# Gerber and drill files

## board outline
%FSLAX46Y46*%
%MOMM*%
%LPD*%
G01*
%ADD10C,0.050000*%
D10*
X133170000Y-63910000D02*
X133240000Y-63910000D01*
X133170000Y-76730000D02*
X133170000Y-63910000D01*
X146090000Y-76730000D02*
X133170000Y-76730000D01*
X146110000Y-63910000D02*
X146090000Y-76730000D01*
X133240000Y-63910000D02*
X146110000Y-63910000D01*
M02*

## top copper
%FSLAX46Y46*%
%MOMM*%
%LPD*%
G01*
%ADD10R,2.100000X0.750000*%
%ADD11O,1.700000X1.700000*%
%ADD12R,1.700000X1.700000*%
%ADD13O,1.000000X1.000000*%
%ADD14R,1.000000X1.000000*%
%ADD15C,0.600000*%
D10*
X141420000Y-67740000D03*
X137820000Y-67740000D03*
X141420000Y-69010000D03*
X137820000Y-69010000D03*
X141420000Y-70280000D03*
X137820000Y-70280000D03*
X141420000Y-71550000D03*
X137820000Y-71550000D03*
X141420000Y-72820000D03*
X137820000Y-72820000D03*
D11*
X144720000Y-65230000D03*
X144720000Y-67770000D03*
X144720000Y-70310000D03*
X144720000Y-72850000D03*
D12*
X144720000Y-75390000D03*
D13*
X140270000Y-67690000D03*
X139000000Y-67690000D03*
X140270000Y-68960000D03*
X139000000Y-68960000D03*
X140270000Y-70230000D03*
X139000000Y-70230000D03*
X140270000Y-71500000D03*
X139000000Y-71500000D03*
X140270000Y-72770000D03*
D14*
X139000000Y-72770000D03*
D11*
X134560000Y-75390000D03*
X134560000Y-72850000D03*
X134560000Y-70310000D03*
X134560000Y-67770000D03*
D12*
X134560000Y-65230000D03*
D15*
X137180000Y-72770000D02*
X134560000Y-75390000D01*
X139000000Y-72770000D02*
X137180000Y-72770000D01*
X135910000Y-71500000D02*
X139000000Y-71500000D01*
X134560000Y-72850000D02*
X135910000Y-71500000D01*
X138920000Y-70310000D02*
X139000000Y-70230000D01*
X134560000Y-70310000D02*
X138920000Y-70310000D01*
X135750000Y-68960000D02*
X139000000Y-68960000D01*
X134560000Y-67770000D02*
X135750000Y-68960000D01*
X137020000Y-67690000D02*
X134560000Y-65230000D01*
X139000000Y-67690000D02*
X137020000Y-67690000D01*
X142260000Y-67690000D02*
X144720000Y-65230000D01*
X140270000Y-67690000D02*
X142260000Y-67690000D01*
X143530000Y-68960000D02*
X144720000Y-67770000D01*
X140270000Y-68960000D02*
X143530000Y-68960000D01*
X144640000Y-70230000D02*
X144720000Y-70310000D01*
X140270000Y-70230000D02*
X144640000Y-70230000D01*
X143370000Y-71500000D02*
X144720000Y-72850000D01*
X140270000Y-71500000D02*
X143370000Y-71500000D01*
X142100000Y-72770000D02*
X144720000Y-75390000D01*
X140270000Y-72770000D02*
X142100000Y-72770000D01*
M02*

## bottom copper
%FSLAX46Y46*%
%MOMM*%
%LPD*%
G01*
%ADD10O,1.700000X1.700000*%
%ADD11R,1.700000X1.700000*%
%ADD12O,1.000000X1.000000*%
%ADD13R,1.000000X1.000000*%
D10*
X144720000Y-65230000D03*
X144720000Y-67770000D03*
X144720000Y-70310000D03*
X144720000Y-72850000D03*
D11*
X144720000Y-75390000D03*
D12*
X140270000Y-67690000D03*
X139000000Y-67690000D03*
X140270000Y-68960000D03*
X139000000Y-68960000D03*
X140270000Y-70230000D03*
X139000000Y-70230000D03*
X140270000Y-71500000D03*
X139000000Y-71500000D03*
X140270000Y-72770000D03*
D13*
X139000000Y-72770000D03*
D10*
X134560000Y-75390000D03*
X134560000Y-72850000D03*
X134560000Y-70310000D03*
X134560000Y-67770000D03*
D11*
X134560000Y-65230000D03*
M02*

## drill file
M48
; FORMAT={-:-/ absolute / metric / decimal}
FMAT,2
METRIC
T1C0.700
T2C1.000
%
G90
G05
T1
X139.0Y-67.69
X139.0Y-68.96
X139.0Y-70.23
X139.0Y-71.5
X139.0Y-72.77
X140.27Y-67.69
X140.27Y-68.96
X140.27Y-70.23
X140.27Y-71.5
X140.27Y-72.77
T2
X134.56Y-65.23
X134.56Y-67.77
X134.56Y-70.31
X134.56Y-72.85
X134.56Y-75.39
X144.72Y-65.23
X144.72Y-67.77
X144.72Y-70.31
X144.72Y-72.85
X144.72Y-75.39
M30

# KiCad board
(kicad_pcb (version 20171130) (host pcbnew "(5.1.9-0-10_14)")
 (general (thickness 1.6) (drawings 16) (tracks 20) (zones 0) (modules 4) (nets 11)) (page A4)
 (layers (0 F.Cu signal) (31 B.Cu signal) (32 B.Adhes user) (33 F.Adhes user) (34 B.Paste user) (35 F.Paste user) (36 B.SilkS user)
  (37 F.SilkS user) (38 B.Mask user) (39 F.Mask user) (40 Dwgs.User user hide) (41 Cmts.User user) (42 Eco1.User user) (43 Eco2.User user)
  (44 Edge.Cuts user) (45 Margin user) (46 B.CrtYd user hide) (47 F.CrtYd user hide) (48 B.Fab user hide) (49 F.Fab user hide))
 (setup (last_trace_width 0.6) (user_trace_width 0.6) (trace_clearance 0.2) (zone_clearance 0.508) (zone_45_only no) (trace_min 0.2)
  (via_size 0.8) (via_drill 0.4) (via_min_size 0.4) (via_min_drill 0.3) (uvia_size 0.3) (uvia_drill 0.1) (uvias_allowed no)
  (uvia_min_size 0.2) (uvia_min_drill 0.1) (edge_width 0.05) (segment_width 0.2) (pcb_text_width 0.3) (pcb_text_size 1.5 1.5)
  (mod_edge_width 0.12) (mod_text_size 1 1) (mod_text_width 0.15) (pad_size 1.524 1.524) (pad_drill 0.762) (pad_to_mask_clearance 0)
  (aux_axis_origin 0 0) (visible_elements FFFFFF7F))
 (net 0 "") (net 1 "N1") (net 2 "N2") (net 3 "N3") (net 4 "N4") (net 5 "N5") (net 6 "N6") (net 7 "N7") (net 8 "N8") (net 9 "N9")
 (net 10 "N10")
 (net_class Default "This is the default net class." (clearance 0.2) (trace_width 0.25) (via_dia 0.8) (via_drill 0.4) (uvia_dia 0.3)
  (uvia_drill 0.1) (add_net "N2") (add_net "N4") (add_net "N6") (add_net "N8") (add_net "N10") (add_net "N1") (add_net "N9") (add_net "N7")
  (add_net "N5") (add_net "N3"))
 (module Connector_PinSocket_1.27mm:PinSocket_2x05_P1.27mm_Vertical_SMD (layer F.Cu) (at 139.62 70.28 180)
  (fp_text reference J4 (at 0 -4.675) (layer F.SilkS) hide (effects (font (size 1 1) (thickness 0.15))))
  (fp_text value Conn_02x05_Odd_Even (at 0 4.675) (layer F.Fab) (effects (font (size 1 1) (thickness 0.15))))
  (pad 10 smd rect (at -1.8 2.54 180) (size 2.1 0.75) (layers F.Cu F.Paste F.Mask) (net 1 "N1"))
  (pad 9 smd rect (at 1.8 2.54 180) (size 2.1 0.75) (layers F.Cu F.Paste F.Mask) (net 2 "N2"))
  (pad 8 smd rect (at -1.8 1.27 180) (size 2.1 0.75) (layers F.Cu F.Paste F.Mask) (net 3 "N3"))
  (pad 7 smd rect (at 1.8 1.27 180) (size 2.1 0.75) (layers F.Cu F.Paste F.Mask) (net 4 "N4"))
  (pad 6 smd rect (at -1.8 0 180) (size 2.1 0.75) (layers F.Cu F.Paste F.Mask) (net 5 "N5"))
  (pad 5 smd rect (at 1.8 0 180) (size 2.1 0.75) (layers F.Cu F.Paste F.Mask) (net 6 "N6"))
  (pad 4 smd rect (at -1.8 -1.27 180) (size 2.1 0.75) (layers F.Cu F.Paste F.Mask) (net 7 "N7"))
  (pad 3 smd rect (at 1.8 -1.27 180) (size 2.1 0.75) (layers F.Cu F.Paste F.Mask) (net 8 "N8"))
  (pad 2 smd rect (at -1.8 -2.54 180) (size 2.1 0.75) (layers F.Cu F.Paste F.Mask) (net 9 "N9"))
  (pad 1 smd rect (at 1.8 -2.54 180) (size 2.1 0.75) (layers F.Cu F.Paste F.Mask) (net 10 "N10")))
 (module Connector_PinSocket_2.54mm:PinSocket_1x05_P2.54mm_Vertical (layer F.Cu) (at 144.72 75.39 180)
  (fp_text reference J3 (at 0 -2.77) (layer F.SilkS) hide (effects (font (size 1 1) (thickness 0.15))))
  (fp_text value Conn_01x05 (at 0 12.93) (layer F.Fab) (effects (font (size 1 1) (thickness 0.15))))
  (pad 5 thru_hole oval (at 0 10.16 180) (size 1.7 1.7) (drill 1) (layers *.Cu *.Mask) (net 1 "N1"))
  (pad 4 thru_hole oval (at 0 7.62 180) (size 1.7 1.7) (drill 1) (layers *.Cu *.Mask) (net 3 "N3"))
  (pad 3 thru_hole oval (at 0 5.08 180) (size 1.7 1.7) (drill 1) (layers *.Cu *.Mask) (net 5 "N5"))
  (pad 2 thru_hole oval (at 0 2.54 180) (size 1.7 1.7) (drill 1) (layers *.Cu *.Mask) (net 7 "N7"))
  (pad 1 thru_hole rect (at 0 0 180) (size 1.7 1.7) (drill 1) (layers *.Cu *.Mask) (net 9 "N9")))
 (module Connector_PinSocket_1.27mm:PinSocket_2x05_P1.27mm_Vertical (layer F.Cu) (at 139 72.77 180)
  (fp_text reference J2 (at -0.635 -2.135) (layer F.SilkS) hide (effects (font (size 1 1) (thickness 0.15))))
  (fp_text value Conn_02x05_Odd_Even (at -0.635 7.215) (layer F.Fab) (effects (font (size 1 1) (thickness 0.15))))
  (pad 10 thru_hole oval (at -1.27 5.08 180) (size 1 1) (drill 0.7) (layers *.Cu *.Mask) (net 1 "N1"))
  (pad 9 thru_hole oval (at 0 5.08 180) (size 1 1) (drill 0.7) (layers *.Cu *.Mask) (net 2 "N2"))
  (pad 8 thru_hole oval (at -1.27 3.81 180) (size 1 1) (drill 0.7) (layers *.Cu *.Mask) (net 3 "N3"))
  (pad 7 thru_hole oval (at 0 3.81 180) (size 1 1) (drill 0.7) (layers *.Cu *.Mask) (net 4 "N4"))
  (pad 6 thru_hole oval (at -1.27 2.54 180) (size 1 1) (drill 0.7) (layers *.Cu *.Mask) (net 5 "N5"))
  (pad 5 thru_hole oval (at 0 2.54 180) (size 1 1) (drill 0.7) (layers *.Cu *.Mask) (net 6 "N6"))
  (pad 4 thru_hole oval (at -1.27 1.27 180) (size 1 1) (drill 0.7) (layers *.Cu *.Mask) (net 7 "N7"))
  (pad 3 thru_hole oval (at 0 1.27 180) (size 1 1) (drill 0.7) (layers *.Cu *.Mask) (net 8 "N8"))
  (pad 2 thru_hole oval (at -1.27 0 180) (size 1 1) (drill 0.7) (layers *.Cu *.Mask) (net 9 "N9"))
  (pad 1 thru_hole rect (at 0 0 180) (size 1 1) (drill 0.7) (layers *.Cu *.Mask) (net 10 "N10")))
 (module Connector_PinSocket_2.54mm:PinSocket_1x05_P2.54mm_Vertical (layer F.Cu) (at 134.56 65.23)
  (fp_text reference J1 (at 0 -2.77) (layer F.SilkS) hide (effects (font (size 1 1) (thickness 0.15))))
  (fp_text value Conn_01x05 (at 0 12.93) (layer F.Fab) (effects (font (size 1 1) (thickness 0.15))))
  (pad 5 thru_hole oval (at 0 10.16) (size 1.7 1.7) (drill 1) (layers *.Cu *.Mask) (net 10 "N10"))
  (pad 4 thru_hole oval (at 0 7.62) (size 1.7 1.7) (drill 1) (layers *.Cu *.Mask) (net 8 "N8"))
  (pad 3 thru_hole oval (at 0 5.08) (size 1.7 1.7) (drill 1) (layers *.Cu *.Mask) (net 6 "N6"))
  (pad 2 thru_hole oval (at 0 2.54) (size 1.7 1.7) (drill 1) (layers *.Cu *.Mask) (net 4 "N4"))
  (pad 1 thru_hole rect (at 0 0) (size 1.7 1.7) (drill 1) (layers *.Cu *.Mask) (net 2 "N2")))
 (gr_line (start 133.17 63.91) (end 133.24 63.91) (layer Edge.Cuts) (width 0.05))
 (gr_line (start 133.17 76.73) (end 133.17 63.91) (layer Edge.Cuts) (width 0.05))
 (gr_line (start 146.09 76.73) (end 133.17 76.73) (layer Edge.Cuts) (width 0.05))
 (gr_line (start 146.11 63.91) (end 146.09 76.73) (layer Edge.Cuts) (width 0.05))
 (gr_line (start 133.24 63.91) (end 146.11 63.91) (layer Edge.Cuts) (width 0.05))
 (segment (start 137.18 72.77) (end 134.56 75.39) (width 0.6) (layer F.Cu) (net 10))
 (segment (start 139 72.77) (end 137.18 72.77) (width 0.6) (layer F.Cu) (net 10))
 (segment (start 135.91 71.5) (end 139 71.5) (width 0.6) (layer F.Cu) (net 8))
 (segment (start 134.56 72.85) (end 135.91 71.5) (width 0.6) (layer F.Cu) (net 8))
 (segment (start 138.92 70.31) (end 139 70.23) (width 0.6) (layer F.Cu) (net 6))
 (segment (start 134.56 70.31) (end 138.92 70.31) (width 0.6) (layer F.Cu) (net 6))
 (segment (start 135.75 68.96) (end 139 68.96) (width 0.6) (layer F.Cu) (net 4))
 (segment (start 134.56 67.77) (end 135.75 68.96) (width 0.6) (layer F.Cu) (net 4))
 (segment (start 137.02 67.69) (end 134.56 65.23) (width 0.6) (layer F.Cu) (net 2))
 (segment (start 139 67.69) (end 137.02 67.69) (width 0.6) (layer F.Cu) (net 2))
 (segment (start 142.26 67.69) (end 144.72 65.23) (width 0.6) (layer F.Cu) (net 1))
 (segment (start 140.27 67.69) (end 142.26 67.69) (width 0.6) (layer F.Cu) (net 1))
 (segment (start 143.53 68.96) (end 144.72 67.77) (width 0.6) (layer F.Cu) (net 3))
 (segment (start 140.27 68.96) (end 143.53 68.96) (width 0.6) (layer F.Cu) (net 3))
 (segment (start 144.64 70.23) (end 144.72 70.31) (width 0.6) (layer F.Cu) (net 5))
 (segment (start 140.27 70.23) (end 144.64 70.23) (width 0.6) (layer F.Cu) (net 5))
 (segment (start 143.37 71.5) (end 144.72 72.85) (width 0.6) (layer F.Cu) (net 7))
 (segment (start 140.27 71.5) (end 143.37 71.5) (width 0.6) (layer F.Cu) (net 7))
 (segment (start 142.1 72.77) (end 144.72 75.39) (width 0.6) (layer F.Cu) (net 9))
 (segment (start 140.27 72.77) (end 142.1 72.77) (width 0.6) (layer F.Cu) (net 9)))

